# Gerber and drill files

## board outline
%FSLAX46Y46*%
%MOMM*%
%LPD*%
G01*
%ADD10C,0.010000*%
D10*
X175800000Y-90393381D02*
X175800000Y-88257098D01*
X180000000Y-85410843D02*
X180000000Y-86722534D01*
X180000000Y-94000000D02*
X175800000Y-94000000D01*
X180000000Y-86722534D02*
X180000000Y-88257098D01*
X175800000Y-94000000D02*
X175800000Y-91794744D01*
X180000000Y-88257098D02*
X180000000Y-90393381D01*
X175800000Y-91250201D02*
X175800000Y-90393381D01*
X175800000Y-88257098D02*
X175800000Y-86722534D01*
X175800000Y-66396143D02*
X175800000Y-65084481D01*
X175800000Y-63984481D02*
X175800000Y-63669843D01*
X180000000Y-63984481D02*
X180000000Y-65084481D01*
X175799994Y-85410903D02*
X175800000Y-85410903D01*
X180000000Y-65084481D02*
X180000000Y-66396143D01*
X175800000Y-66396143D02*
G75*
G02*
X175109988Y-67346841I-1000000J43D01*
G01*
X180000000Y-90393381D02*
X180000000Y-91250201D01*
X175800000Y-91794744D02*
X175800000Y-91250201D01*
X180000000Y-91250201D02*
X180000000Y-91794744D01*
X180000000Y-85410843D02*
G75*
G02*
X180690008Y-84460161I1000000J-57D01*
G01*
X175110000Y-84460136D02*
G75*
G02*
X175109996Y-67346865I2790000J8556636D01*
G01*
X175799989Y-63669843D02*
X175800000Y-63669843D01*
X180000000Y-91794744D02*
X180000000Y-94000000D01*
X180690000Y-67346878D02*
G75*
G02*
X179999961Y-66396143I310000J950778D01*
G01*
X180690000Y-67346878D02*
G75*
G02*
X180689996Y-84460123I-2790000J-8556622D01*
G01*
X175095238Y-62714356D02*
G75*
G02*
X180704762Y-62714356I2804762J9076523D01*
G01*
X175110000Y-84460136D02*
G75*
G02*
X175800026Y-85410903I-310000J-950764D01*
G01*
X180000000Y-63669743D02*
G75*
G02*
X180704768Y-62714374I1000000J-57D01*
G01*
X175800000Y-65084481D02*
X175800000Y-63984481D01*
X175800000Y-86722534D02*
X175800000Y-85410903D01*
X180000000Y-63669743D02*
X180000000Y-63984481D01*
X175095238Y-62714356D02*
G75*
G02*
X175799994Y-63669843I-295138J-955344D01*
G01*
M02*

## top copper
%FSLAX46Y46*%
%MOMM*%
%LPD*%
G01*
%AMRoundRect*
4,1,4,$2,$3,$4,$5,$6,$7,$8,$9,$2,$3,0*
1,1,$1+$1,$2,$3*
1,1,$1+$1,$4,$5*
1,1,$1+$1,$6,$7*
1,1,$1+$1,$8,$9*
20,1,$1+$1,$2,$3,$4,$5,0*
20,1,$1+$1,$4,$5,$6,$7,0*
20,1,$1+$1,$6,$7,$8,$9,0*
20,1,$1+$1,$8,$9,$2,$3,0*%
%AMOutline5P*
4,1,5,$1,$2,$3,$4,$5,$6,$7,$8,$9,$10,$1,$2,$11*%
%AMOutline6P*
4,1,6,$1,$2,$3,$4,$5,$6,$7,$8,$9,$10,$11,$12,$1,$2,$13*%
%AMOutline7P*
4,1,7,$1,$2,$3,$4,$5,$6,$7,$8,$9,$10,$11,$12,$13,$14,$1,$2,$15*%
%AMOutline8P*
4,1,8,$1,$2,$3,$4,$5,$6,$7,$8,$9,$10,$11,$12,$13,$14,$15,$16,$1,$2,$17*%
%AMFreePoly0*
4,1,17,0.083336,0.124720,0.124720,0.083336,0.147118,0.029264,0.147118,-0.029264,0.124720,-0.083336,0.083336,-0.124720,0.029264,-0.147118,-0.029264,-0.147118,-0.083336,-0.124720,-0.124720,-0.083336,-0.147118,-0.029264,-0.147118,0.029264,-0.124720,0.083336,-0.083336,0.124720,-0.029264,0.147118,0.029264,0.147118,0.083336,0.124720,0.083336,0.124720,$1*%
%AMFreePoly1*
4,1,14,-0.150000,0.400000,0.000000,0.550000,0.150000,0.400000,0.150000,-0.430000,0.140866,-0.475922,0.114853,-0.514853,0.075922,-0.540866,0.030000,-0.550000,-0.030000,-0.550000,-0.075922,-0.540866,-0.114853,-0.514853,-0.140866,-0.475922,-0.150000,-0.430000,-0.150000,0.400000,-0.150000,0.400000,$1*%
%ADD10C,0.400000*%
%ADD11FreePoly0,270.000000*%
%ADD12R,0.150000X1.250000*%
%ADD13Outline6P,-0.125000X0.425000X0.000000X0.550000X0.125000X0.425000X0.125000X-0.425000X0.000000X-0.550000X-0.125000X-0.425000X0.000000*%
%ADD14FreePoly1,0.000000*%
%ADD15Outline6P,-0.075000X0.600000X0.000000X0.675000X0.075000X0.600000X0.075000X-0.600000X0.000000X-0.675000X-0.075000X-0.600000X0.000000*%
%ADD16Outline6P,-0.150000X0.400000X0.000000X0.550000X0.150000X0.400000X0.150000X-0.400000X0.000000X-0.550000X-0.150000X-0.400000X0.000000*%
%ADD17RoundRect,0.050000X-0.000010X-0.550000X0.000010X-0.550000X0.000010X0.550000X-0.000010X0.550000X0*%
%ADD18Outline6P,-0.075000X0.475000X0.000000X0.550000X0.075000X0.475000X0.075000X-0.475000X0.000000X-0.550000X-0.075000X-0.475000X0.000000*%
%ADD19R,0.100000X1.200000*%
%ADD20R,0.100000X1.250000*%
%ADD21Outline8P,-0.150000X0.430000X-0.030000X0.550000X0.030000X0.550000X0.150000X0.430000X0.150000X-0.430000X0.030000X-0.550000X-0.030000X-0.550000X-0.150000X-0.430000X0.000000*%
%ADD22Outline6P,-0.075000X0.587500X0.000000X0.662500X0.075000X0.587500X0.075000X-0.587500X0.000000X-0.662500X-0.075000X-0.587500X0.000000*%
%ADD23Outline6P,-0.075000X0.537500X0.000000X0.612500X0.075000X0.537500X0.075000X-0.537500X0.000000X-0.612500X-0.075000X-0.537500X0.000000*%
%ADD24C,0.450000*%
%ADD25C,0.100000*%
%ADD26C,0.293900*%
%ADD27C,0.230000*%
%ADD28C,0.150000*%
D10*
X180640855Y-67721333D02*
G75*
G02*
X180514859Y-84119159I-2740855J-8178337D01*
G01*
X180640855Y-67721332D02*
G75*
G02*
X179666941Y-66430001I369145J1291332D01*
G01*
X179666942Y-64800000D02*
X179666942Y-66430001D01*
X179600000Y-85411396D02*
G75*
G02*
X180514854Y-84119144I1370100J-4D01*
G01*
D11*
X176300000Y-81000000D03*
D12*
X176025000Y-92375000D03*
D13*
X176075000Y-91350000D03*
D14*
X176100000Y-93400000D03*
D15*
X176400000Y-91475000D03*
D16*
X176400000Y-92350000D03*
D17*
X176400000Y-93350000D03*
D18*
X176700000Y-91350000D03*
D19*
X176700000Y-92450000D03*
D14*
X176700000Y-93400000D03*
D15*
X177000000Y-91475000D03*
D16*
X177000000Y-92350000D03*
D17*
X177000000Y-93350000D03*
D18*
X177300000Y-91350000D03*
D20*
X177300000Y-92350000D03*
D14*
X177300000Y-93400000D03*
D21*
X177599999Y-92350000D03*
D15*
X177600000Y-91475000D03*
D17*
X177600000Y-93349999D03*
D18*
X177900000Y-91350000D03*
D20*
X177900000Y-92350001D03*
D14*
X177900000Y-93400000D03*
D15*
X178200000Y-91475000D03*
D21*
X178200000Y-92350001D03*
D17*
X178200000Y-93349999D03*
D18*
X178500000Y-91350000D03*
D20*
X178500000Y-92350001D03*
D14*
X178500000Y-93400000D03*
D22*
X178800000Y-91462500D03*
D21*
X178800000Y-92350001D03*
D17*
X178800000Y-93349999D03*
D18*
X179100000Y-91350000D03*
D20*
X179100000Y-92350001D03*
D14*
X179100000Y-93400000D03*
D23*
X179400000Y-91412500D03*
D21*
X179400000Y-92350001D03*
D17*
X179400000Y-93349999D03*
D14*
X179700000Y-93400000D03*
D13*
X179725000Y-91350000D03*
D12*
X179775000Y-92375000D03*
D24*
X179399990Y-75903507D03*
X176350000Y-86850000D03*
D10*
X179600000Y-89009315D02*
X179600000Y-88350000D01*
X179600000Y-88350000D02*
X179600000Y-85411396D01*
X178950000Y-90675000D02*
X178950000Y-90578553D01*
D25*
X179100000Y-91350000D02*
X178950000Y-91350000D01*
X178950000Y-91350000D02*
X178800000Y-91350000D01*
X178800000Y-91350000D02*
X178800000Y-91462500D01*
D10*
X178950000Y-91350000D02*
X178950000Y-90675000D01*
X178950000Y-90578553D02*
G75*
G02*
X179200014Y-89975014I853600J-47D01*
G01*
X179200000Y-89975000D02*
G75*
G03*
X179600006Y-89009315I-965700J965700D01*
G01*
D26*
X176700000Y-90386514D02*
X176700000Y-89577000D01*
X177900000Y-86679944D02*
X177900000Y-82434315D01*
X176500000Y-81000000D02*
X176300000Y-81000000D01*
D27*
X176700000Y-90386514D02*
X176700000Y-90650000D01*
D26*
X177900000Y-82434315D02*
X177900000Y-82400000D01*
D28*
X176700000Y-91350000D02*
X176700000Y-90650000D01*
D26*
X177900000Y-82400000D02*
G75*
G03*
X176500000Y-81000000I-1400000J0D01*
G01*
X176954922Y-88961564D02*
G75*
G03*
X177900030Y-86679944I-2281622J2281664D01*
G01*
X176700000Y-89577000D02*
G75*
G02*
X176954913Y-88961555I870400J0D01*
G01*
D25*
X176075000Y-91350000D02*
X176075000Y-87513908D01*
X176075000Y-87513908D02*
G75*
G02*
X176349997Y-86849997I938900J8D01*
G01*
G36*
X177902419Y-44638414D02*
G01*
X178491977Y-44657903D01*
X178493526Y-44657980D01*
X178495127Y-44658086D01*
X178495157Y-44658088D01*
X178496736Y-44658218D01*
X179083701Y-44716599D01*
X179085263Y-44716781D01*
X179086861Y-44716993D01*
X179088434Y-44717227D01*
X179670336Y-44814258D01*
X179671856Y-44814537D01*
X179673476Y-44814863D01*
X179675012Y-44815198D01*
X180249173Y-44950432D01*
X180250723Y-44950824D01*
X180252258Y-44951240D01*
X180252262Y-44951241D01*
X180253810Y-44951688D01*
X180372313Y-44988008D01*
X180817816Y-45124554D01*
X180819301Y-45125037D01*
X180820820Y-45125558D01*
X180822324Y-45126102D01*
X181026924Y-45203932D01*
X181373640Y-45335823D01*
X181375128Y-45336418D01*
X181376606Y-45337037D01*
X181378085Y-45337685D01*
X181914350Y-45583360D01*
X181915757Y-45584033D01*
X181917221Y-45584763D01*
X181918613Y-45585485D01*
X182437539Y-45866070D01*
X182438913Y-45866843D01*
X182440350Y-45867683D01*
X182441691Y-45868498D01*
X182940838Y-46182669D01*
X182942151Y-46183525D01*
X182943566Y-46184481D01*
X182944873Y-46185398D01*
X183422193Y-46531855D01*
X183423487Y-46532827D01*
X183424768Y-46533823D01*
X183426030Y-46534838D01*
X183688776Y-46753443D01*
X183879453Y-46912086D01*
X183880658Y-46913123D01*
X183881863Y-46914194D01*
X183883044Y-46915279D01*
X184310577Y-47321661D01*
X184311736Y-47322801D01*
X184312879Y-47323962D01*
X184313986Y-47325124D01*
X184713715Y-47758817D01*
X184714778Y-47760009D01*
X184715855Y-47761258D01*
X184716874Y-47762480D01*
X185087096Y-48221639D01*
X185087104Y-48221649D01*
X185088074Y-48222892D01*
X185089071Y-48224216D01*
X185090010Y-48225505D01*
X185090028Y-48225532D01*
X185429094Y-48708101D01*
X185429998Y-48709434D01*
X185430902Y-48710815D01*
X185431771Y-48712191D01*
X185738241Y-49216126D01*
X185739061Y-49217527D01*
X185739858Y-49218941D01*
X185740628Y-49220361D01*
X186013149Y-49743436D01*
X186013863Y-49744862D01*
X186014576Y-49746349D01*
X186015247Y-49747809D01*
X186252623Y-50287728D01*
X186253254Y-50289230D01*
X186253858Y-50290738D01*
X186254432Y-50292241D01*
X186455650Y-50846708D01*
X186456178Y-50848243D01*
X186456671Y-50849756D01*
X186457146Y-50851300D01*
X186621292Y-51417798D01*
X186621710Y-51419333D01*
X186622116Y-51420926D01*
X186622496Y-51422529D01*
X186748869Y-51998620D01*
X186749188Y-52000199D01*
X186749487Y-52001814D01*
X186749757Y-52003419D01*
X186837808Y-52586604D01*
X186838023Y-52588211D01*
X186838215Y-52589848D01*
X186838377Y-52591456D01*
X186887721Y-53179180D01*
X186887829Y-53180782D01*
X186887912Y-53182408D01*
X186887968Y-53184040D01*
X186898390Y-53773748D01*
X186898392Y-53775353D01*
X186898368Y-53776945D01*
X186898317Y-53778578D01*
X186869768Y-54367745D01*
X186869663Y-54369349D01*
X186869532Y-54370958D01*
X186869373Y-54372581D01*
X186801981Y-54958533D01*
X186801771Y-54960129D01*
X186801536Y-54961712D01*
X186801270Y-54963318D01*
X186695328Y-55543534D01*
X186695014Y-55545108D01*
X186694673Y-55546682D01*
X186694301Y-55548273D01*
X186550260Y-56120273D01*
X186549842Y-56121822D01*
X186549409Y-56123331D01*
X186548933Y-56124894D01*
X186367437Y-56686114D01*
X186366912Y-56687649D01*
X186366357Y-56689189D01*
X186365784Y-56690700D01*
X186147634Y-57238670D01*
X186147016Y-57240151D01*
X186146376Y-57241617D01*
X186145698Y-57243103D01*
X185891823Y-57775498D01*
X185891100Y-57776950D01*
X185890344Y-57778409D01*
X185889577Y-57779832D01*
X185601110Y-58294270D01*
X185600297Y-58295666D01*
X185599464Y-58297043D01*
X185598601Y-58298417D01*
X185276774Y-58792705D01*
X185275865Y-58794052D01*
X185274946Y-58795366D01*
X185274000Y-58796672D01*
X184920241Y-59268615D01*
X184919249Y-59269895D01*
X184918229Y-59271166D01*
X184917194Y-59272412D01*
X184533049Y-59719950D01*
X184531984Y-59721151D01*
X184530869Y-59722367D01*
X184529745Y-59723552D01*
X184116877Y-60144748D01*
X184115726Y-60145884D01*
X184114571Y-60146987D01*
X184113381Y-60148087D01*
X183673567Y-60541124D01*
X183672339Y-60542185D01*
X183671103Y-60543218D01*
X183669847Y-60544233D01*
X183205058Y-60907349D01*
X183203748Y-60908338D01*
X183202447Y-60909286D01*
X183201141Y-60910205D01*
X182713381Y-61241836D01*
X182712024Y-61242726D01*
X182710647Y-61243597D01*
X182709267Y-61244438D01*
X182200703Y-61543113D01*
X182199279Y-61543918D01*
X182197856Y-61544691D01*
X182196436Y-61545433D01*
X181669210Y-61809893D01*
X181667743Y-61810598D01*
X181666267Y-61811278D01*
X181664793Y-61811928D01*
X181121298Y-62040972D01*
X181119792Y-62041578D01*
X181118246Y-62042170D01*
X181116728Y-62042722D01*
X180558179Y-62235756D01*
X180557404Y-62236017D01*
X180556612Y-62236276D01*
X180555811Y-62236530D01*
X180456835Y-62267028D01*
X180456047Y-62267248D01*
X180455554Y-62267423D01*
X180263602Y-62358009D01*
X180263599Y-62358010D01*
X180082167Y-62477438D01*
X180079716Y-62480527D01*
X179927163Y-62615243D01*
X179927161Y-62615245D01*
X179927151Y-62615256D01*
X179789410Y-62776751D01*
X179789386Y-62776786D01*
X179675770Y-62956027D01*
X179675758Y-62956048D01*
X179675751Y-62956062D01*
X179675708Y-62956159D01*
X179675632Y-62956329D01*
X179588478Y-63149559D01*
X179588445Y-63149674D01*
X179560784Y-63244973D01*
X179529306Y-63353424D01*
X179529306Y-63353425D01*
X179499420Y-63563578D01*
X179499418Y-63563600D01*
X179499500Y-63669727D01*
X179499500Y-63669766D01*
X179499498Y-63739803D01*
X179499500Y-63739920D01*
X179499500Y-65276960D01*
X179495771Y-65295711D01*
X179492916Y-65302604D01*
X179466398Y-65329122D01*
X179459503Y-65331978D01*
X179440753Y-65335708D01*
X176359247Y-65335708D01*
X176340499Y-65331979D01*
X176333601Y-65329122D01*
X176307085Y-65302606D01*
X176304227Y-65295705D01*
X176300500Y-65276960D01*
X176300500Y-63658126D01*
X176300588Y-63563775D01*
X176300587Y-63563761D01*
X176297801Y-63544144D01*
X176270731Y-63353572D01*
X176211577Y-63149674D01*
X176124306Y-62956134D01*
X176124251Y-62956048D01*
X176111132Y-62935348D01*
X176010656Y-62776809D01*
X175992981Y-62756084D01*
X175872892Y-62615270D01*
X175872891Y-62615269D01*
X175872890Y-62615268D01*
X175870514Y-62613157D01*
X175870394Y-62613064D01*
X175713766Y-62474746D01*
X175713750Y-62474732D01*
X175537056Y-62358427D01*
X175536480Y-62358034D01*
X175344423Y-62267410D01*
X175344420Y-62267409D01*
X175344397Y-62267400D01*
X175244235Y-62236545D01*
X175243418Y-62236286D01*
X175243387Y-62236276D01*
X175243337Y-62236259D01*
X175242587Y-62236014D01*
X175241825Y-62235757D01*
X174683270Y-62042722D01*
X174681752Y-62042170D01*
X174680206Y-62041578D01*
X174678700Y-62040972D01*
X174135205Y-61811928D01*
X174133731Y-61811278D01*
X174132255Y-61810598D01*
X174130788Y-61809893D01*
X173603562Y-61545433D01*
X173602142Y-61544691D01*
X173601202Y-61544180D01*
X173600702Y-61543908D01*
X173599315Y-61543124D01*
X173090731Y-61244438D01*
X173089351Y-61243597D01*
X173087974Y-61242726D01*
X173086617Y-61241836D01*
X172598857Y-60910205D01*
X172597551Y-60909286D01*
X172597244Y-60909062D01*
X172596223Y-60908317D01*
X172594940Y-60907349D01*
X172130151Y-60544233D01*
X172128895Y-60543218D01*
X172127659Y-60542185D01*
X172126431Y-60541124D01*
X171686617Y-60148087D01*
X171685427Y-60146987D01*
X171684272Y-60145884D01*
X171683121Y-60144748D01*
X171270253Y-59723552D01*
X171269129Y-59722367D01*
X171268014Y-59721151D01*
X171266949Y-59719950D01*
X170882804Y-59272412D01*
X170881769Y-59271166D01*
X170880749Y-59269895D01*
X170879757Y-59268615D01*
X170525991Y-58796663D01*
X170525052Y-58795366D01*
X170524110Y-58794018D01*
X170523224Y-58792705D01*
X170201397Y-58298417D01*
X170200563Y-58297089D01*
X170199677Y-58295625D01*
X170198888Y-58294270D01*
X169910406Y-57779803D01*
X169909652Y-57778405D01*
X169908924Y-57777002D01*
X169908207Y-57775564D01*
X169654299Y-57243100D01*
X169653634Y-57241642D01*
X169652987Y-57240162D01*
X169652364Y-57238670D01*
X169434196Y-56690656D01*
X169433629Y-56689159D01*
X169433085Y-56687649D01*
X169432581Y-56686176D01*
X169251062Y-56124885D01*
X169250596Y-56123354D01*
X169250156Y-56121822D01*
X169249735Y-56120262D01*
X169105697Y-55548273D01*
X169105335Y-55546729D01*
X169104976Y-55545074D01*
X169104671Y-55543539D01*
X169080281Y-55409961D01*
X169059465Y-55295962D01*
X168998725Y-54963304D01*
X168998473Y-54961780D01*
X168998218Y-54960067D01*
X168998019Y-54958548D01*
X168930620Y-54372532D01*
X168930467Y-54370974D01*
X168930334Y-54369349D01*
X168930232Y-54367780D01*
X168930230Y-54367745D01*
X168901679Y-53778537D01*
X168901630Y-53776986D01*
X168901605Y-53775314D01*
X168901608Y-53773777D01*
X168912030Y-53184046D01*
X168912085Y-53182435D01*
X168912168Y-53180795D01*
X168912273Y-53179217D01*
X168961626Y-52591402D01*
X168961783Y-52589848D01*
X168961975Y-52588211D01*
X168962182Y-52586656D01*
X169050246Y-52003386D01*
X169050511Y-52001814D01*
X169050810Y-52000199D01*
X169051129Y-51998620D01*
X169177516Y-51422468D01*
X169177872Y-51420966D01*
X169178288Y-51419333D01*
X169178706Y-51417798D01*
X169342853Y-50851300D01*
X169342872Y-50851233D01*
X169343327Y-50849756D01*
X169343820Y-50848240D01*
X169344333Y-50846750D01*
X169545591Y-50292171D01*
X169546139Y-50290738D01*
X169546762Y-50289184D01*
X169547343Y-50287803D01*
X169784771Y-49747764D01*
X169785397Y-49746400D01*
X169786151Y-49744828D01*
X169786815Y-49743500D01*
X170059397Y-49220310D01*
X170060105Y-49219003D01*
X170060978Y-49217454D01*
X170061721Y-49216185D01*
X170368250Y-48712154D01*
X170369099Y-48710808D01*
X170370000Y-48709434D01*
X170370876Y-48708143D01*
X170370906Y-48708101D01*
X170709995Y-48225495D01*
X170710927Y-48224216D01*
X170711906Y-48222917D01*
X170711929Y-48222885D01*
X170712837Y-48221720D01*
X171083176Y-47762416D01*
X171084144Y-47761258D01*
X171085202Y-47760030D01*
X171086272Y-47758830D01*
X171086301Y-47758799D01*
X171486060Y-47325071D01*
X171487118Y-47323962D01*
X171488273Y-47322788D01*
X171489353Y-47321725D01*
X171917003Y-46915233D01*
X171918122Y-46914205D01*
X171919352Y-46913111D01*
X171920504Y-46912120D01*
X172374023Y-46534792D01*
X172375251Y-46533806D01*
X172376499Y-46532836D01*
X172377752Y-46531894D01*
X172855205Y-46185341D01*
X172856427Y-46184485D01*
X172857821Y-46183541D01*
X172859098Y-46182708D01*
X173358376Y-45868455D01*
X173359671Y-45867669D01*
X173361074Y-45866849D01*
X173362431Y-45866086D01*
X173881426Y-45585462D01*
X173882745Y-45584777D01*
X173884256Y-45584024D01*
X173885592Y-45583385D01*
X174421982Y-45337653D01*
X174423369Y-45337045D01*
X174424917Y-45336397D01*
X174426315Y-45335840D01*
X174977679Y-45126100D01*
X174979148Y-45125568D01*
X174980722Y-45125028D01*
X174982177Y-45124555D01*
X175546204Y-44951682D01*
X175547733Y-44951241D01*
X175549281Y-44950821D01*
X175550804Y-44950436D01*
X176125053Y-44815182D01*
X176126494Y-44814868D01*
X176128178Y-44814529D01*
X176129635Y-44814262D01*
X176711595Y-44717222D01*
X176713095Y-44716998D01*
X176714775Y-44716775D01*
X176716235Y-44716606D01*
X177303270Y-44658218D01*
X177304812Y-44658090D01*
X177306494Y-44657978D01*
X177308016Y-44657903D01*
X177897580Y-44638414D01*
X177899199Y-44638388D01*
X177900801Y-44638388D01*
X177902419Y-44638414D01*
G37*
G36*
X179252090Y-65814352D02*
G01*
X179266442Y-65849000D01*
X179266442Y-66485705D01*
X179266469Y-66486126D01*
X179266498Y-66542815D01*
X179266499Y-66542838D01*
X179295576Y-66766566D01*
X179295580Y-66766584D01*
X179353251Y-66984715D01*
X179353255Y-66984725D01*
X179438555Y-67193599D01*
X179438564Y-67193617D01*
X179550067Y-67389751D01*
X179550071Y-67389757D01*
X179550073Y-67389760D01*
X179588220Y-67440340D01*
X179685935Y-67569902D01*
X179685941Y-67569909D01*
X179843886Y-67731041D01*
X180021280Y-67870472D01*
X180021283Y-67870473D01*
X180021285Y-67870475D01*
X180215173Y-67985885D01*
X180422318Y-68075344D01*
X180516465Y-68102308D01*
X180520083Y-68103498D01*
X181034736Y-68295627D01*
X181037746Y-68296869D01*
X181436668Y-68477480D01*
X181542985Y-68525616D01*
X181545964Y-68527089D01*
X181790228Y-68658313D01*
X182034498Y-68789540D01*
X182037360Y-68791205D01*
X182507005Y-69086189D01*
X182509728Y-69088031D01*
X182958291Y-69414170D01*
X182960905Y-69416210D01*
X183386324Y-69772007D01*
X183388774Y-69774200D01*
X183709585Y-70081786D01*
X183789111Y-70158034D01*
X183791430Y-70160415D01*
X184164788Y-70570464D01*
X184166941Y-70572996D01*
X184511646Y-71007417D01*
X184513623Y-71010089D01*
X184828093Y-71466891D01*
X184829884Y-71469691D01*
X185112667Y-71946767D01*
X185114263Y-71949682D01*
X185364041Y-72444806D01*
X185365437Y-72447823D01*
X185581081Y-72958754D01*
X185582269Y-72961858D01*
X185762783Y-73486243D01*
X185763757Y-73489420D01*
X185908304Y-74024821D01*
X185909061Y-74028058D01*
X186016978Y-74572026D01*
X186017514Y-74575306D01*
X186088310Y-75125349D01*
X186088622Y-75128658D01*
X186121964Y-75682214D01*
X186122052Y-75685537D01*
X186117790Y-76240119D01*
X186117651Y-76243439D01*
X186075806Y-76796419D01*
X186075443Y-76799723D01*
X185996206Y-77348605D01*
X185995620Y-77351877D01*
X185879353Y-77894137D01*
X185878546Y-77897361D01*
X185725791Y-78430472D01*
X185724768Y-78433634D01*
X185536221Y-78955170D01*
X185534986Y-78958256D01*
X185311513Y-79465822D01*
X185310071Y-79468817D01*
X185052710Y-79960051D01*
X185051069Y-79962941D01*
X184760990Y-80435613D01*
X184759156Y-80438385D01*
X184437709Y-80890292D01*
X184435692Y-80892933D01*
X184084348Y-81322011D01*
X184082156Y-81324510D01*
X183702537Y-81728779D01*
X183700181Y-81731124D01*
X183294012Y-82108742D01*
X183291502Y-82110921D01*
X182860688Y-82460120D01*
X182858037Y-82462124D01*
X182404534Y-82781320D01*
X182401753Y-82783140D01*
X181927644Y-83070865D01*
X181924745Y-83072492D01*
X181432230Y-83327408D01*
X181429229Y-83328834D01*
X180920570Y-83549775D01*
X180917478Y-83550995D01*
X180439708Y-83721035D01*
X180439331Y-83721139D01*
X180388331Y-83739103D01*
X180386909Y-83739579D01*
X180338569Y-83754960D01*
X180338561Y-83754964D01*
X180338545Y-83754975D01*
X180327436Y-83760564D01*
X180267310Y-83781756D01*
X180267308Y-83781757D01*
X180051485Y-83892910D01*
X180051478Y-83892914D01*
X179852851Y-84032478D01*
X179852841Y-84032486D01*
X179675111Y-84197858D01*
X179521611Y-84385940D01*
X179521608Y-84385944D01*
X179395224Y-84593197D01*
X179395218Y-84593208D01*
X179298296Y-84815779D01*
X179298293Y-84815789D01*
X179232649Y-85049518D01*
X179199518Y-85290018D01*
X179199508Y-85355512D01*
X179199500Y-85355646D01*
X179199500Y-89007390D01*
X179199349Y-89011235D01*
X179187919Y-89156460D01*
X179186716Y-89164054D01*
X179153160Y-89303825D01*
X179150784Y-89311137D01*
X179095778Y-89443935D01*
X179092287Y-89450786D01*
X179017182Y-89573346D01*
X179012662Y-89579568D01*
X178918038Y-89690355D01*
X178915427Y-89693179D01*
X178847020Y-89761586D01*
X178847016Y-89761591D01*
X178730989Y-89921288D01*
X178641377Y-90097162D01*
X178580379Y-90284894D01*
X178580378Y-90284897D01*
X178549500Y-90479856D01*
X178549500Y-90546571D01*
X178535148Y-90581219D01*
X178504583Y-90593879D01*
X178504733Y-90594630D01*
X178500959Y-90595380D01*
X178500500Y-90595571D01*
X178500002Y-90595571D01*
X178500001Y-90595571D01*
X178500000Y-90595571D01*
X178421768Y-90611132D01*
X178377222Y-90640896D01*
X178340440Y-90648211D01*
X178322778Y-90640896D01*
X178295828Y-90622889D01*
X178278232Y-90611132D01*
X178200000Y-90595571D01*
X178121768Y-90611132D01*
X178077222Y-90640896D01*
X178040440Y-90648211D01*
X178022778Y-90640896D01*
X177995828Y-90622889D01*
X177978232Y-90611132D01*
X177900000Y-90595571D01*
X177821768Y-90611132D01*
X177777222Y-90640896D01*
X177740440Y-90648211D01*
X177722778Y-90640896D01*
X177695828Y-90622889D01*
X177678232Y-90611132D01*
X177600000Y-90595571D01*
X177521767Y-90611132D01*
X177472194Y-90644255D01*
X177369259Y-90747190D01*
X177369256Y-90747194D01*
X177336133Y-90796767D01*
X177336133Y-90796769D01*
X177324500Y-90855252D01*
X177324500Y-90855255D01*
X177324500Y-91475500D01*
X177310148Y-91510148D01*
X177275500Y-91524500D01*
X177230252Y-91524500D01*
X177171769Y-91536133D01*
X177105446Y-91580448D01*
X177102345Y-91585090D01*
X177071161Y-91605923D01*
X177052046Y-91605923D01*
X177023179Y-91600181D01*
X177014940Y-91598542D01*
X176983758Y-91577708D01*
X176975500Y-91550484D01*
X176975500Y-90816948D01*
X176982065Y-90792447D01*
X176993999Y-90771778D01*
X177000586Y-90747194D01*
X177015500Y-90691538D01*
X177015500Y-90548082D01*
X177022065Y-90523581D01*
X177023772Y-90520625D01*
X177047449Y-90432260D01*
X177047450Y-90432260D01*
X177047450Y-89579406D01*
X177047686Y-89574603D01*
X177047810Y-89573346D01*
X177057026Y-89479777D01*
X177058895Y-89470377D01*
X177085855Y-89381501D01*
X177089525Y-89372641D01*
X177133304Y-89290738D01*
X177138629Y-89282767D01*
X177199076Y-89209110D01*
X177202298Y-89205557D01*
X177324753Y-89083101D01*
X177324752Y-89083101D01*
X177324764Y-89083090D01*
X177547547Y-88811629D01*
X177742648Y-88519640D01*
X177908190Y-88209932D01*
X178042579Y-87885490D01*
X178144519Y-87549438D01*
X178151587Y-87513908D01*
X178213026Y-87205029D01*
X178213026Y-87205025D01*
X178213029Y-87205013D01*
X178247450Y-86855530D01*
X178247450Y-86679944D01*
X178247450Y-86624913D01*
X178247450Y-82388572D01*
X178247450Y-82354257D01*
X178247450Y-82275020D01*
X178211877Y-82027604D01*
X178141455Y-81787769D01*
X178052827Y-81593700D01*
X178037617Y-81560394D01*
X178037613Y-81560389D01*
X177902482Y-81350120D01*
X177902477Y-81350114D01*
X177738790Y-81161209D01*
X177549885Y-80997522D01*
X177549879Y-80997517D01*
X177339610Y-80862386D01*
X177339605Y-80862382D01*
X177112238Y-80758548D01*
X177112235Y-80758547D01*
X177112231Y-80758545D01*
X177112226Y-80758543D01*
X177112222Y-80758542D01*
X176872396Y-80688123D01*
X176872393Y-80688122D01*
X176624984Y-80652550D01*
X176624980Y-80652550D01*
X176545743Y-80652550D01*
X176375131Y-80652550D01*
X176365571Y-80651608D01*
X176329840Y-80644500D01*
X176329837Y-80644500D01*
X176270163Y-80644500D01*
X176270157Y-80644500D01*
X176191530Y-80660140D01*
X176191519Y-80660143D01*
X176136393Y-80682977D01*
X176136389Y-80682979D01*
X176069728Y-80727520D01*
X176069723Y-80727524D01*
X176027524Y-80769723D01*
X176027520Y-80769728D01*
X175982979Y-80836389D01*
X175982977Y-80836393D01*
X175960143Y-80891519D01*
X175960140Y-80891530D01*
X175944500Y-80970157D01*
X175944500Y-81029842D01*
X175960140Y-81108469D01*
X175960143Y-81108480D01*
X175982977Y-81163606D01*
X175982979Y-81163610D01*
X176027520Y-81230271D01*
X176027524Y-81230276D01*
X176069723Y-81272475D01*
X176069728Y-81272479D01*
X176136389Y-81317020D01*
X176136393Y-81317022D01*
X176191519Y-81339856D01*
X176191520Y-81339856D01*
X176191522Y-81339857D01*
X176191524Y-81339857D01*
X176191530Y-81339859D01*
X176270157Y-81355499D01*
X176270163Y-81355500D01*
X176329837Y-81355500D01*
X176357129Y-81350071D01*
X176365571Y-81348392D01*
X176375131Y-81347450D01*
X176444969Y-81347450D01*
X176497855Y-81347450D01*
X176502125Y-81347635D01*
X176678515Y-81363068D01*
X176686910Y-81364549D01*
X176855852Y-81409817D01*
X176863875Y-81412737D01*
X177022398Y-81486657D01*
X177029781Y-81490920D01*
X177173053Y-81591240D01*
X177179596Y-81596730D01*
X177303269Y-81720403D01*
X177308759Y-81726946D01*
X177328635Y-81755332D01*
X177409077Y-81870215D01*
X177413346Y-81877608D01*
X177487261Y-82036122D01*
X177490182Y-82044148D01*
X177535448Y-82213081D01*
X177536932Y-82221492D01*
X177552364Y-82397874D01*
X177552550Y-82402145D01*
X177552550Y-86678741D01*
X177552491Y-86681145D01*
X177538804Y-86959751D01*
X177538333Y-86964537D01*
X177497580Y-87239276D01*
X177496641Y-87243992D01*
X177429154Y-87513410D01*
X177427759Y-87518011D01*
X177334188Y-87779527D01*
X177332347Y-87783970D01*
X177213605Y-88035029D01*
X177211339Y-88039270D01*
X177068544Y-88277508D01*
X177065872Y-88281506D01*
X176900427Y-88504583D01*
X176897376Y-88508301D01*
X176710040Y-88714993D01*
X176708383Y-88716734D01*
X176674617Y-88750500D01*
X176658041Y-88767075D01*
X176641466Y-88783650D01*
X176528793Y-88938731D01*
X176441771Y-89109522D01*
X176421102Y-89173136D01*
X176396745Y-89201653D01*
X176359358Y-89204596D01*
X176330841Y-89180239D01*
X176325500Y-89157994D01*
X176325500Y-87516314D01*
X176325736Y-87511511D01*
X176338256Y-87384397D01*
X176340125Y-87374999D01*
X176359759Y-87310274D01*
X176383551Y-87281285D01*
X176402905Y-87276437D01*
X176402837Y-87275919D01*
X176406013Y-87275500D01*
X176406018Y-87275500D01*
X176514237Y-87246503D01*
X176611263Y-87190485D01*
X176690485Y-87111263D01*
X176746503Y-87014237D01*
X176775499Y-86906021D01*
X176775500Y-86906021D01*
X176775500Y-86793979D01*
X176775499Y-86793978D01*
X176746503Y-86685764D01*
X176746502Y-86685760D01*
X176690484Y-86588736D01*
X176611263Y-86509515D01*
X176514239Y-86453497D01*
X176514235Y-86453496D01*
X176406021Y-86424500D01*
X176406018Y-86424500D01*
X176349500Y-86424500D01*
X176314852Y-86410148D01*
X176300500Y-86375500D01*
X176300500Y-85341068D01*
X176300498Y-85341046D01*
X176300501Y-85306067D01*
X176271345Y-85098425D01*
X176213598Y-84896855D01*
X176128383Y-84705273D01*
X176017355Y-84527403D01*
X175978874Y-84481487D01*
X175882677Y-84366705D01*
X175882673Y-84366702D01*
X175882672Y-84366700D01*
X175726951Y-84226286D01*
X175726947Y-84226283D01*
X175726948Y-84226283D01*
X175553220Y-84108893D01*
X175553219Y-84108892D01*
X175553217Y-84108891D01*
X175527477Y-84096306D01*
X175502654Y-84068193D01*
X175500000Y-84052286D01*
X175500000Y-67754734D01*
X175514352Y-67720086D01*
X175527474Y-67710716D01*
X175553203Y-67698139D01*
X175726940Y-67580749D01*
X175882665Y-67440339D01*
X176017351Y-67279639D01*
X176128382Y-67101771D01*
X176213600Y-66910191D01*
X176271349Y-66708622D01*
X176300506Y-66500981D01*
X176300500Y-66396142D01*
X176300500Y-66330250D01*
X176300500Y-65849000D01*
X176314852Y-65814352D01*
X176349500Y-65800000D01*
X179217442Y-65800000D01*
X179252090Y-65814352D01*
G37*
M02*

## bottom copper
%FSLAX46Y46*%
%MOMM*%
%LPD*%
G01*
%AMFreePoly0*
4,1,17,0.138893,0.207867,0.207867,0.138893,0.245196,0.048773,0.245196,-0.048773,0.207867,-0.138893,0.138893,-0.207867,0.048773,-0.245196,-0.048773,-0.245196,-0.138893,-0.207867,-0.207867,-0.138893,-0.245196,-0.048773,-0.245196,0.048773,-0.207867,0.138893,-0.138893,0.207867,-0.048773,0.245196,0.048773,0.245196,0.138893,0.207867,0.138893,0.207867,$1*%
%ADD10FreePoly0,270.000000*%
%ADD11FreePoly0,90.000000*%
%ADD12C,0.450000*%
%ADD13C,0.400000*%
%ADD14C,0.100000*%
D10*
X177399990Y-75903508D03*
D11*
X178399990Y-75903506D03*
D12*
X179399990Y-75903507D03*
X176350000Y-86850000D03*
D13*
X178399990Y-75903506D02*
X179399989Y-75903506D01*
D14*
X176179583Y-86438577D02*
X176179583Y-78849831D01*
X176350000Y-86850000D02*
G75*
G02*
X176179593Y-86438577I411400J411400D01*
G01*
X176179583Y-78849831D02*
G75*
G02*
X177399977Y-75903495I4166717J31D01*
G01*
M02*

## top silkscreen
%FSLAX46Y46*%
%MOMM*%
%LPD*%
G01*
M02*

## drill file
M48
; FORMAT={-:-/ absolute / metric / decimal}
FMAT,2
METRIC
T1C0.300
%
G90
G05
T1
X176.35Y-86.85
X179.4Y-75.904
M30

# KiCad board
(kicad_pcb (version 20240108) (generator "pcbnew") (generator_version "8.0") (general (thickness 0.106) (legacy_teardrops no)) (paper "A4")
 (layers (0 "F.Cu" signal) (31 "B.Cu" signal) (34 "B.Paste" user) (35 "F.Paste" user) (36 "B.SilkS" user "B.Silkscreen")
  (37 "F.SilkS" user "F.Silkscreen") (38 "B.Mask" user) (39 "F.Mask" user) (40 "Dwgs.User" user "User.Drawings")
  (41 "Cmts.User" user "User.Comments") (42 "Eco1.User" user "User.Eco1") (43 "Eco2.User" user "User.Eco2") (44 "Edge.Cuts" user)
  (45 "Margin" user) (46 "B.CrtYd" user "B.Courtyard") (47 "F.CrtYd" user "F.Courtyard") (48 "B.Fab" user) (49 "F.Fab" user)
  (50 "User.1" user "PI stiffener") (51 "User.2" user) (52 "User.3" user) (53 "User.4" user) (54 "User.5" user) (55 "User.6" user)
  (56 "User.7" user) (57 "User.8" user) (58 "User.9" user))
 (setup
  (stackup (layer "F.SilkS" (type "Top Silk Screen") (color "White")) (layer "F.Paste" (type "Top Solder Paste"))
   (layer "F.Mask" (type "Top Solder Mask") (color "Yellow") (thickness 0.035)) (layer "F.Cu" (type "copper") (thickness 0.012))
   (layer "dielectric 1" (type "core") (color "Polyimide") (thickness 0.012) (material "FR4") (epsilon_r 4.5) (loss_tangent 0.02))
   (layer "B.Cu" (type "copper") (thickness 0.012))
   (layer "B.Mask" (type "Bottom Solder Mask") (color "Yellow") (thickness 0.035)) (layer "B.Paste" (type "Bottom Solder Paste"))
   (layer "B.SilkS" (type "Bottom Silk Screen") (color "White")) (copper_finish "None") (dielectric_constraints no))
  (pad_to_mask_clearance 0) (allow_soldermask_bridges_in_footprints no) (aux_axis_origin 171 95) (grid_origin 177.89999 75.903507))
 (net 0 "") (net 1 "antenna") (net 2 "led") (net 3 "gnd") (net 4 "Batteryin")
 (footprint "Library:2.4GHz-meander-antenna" (layer "F.Cu") (at 176.3 81 -90)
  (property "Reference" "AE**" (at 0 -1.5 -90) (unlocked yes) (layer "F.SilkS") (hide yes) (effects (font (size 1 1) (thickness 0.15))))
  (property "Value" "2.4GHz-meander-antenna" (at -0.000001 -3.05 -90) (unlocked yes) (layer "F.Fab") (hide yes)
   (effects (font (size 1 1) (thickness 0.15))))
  (pad "1" smd custom (at 0 0 270) (size 0.3 0.3) (layers "F.Cu") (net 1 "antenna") (thermal_bridge_angle 90)
   (options (clearance outline) (anchor circle)) (primitives)))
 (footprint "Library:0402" (layer "B.Cu") (at 177.89999 75.903507)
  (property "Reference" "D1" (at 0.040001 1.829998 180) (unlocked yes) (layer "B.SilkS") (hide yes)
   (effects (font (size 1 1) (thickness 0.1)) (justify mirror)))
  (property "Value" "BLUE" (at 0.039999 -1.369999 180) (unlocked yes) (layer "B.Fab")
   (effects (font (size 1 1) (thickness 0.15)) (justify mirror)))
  (pad "1" smd custom (at -0.5 0.000001 270) (size 0.5 0.5) (layers "B.Cu" "B.Paste" "B.Mask") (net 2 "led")
   (options (clearance outline) (anchor circle)) (primitives))
  (pad "2" smd custom (at 0.5 -0.000001 90) (size 0.5 0.5) (layers "B.Cu" "B.Paste" "B.Mask") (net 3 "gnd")
   (options (clearance outline) (anchor circle)) (primitives)))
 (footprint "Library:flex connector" (layer "B.Cu") (at 175.7 90.05)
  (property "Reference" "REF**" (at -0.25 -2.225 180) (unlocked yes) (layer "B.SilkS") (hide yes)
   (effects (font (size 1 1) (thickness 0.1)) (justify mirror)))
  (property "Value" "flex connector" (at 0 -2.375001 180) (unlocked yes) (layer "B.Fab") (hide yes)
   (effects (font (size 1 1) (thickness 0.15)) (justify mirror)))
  (pad "1" smd rect (at 0.325 2.325) (size 0.15 1.25) (layers "F.Cu" "F.Paste" "F.Mask") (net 2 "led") (thermal_bridge_angle 45))
  (pad "1" smd roundrect (at 0.375 1.3) (size 0.25 1.1) (layers "F.Cu" "F.Paste" "F.Mask") (roundrect_rratio 0) (chamfer_ratio 0.5)
   (chamfer top_left top_right bottom_left bottom_right) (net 2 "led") (thermal_bridge_angle 45))
  (pad "1" smd roundrect (at 0.4 3.35) (size 0.3 1.1) (layers "F.Cu" "F.Paste" "F.Mask") (roundrect_rratio 0.4) (chamfer_ratio 0.5)
   (chamfer top_left top_right) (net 2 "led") (thermal_bridge_angle 45))
  (pad "2" smd roundrect (at 0.7 1.425) (size 0.15 1.35) (layers "F.Cu" "F.Paste" "F.Mask") (roundrect_rratio 0) (chamfer_ratio 0.5)
   (chamfer top_left top_right bottom_left bottom_right) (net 3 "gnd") (thermal_bridge_angle 45))
  (pad "2" smd roundrect (at 0.7 2.3) (size 0.3 1.1) (layers "F.Cu" "F.Paste" "F.Mask") (roundrect_rratio 0) (chamfer_ratio 0.5)
   (chamfer top_left top_right bottom_left bottom_right) (thermal_bridge_angle 45))
  (pad "2" smd roundrect (at 0.7 3.3) (size 0.1 1.2) (layers "F.Cu" "F.Paste" "F.Mask") (roundrect_rratio 0.5) (thermal_bridge_angle 45))
  (pad "3" smd roundrect (at 1 1.3) (size 0.15 1.1) (layers "F.Cu" "F.Paste" "F.Mask") (roundrect_rratio 0) (chamfer_ratio 0.5)
   (chamfer top_left top_right bottom_left bottom_right) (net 1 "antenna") (thermal_bridge_angle 45))
  (pad "3" smd rect (at 1 2.4) (size 0.1 1.2) (layers "F.Cu" "F.Paste" "F.Mask") (thermal_bridge_angle 45))
  (pad "3" smd roundrect (at 1 3.35) (size 0.3 1.1) (layers "F.Cu" "F.Paste" "F.Mask") (roundrect_rratio 0.4) (chamfer_ratio 0.5)
   (chamfer top_left top_right) (thermal_bridge_angle 45))
  (pad "4" smd roundrect (at 1.3 1.425) (size 0.15 1.35) (layers "F.Cu" "F.Paste" "F.Mask") (roundrect_rratio 0) (chamfer_ratio 0.5)
   (chamfer top_left top_right bottom_left bottom_right) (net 3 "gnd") (thermal_bridge_angle 45))
  (pad "4" smd roundrect (at 1.3 2.3) (size 0.3 1.1) (layers "F.Cu" "F.Paste" "F.Mask") (roundrect_rratio 0) (chamfer_ratio 0.5)
   (chamfer top_left top_right bottom_left bottom_right) (thermal_bridge_angle 45))
  (pad "4" smd roundrect (at 1.3 3.3) (size 0.1 1.2) (layers "F.Cu" "F.Paste" "F.Mask") (roundrect_rratio 0.5) (thermal_bridge_angle 45))
  (pad "5" smd roundrect (at 1.6 1.3) (size 0.15 1.1) (layers "F.Cu" "F.Paste" "F.Mask") (roundrect_rratio 0) (chamfer_ratio 0.5)
   (chamfer top_left top_right bottom_left bottom_right) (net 3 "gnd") (thermal_bridge_angle 45))
  (pad "5" smd rect (at 1.6 2.3) (size 0.1 1.25) (layers "F.Cu" "F.Paste" "F.Mask") (thermal_bridge_angle 45))
  (pad "5" smd roundrect (at 1.6 3.35) (size 0.3 1.1) (layers "F.Cu" "F.Paste" "F.Mask") (roundrect_rratio 0.4) (chamfer_ratio 0.5)
   (chamfer top_left top_right) (thermal_bridge_angle 45))
  (pad "6" smd roundrect (at 1.899999 2.3) (size 0.3 1.1) (layers "F.Cu" "F.Paste" "F.Mask") (roundrect_rratio 0) (chamfer_ratio 0.4)
   (chamfer top_left top_right bottom_left bottom_right) (thermal_bridge_angle 45))
  (pad "6" smd roundrect (at 1.9 1.425) (size 0.15 1.35) (layers "F.Cu" "F.Paste" "F.Mask") (roundrect_rratio 0) (chamfer_ratio 0.5)
   (chamfer top_left top_right bottom_left bottom_right) (thermal_bridge_angle 45))
  (pad "6" smd roundrect (at 1.9 3.299999) (size 0.1 1.2) (layers "F.Cu" "F.Paste" "F.Mask") (roundrect_rratio 0.5)
   (thermal_bridge_angle 45))
  (pad "7" smd roundrect (at 2.2 1.3) (size 0.15 1.1) (layers "F.Cu" "F.Paste" "F.Mask") (roundrect_rratio 0) (chamfer_ratio 0.5)
   (chamfer top_left top_right bottom_left bottom_right) (thermal_bridge_angle 45))
  (pad "7" smd rect (at 2.2 2.300001) (size 0.1 1.25) (layers "F.Cu" "F.Paste" "F.Mask") (thermal_bridge_angle 45))
  (pad "7" smd roundrect (at 2.2 3.35) (size 0.3 1.1) (layers "F.Cu" "F.Paste" "F.Mask") (roundrect_rratio 0.4) (chamfer_ratio 0.5)
   (chamfer top_left top_right) (thermal_bridge_angle 45))
  (pad "8" smd roundrect (at 2.5 1.425) (size 0.15 1.35) (layers "F.Cu" "F.Paste" "F.Mask") (roundrect_rratio 0) (chamfer_ratio 0.5)
   (chamfer top_left top_right bottom_left bottom_right) (thermal_bridge_angle 45))
  (pad "8" smd roundrect (at 2.5 2.300001) (size 0.3 1.1) (layers "F.Cu" "F.Paste" "F.Mask") (roundrect_rratio 0) (chamfer_ratio 0.4)
   (chamfer top_left top_right bottom_left bottom_right) (thermal_bridge_angle 45))
  (pad "8" smd roundrect (at 2.5 3.299999) (size 0.1 1.2) (layers "F.Cu" "F.Paste" "F.Mask") (roundrect_rratio 0.5)
   (thermal_bridge_angle 45))
  (pad "9" smd roundrect (at 2.8 1.3) (size 0.15 1.1) (layers "F.Cu" "F.Paste" "F.Mask") (roundrect_rratio 0) (chamfer_ratio 0.5)
   (chamfer top_left top_right bottom_left bottom_right) (thermal_bridge_angle 45))
  (pad "9" smd rect (at 2.8 2.300001) (size 0.1 1.25) (layers "F.Cu" "F.Paste" "F.Mask") (thermal_bridge_angle 45))
  (pad "9" smd roundrect (at 2.8 3.35) (size 0.3 1.1) (layers "F.Cu" "F.Paste" "F.Mask") (roundrect_rratio 0.4) (chamfer_ratio 0.5)
   (chamfer top_left top_right) (thermal_bridge_angle 45))
  (pad "10" smd roundrect (at 3.1 1.4125) (size 0.15 1.325) (layers "F.Cu" "F.Paste" "F.Mask") (roundrect_rratio 0) (chamfer_ratio 0.5)
   (chamfer top_left top_right bottom_left bottom_right) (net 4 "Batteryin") (thermal_bridge_angle 45))
  (pad "10" smd roundrect (at 3.1 2.300001) (size 0.3 1.1) (layers "F.Cu" "F.Paste" "F.Mask") (roundrect_rratio 0) (chamfer_ratio 0.4)
   (chamfer top_left top_right bottom_left bottom_right) (thermal_bridge_angle 45))
  (pad "10" smd roundrect (at 3.1 3.299999) (size 0.1 1.2) (layers "F.Cu" "F.Paste" "F.Mask") (roundrect_rratio 0.5)
   (thermal_bridge_angle 45))
  (pad "11" smd roundrect (at 3.4 1.3) (size 0.15 1.1) (layers "F.Cu" "F.Paste" "F.Mask") (roundrect_rratio 0) (chamfer_ratio 0.5)
   (chamfer top_left top_right bottom_left bottom_right) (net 4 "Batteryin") (thermal_bridge_angle 45))
  (pad "11" smd rect (at 3.4 2.300001) (size 0.1 1.25) (layers "F.Cu" "F.Paste" "F.Mask") (thermal_bridge_angle 45))
  (pad "11" smd roundrect (at 3.4 3.35) (size 0.3 1.1) (layers "F.Cu" "F.Paste" "F.Mask") (roundrect_rratio 0.4) (chamfer_ratio 0.5)
   (chamfer top_left top_right) (thermal_bridge_angle 45))
  (pad "12" smd roundrect (at 3.7 1.3625) (size 0.15 1.225) (layers "F.Cu" "F.Paste" "F.Mask") (roundrect_rratio 0) (chamfer_ratio 0.5)
   (chamfer top_left top_right bottom_left bottom_right) (thermal_bridge_angle 45))
  (pad "12" smd roundrect (at 3.7 2.300001) (size 0.3 1.1) (layers "F.Cu" "F.Paste" "F.Mask") (roundrect_rratio 0) (chamfer_ratio 0.4)
   (chamfer top_left top_right bottom_left bottom_right) (thermal_bridge_angle 45))
  (pad "12" smd roundrect (at 3.7 3.299999) (size 0.1 1.2) (layers "F.Cu" "F.Paste" "F.Mask") (roundrect_rratio 0.5)
   (thermal_bridge_angle 45))
  (pad "13" smd roundrect (at 4 3.35) (size 0.3 1.1) (layers "F.Cu" "F.Paste" "F.Mask") (roundrect_rratio 0.4) (chamfer_ratio 0.5)
   (chamfer top_left top_right) (thermal_bridge_angle 45))
  (pad "13" smd roundrect (at 4.025 1.3) (size 0.25 1.1) (layers "F.Cu" "F.Paste" "F.Mask") (roundrect_rratio 0) (chamfer_ratio 0.5)
   (chamfer top_left top_right bottom_left bottom_right) (thermal_bridge_angle 45))
  (pad "13" smd rect (at 4.075 2.325) (size 0.15 1.25) (layers "F.Cu" "F.Paste" "F.Mask") (thermal_bridge_angle 45)))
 (gr_arc (start 180.640855 67.721333) (mid 186.525141 75.965942) (end 180.514858 84.119155) (stroke (width 0.4) (type default))
  (layer "F.Cu") (net 4))
 (gr_arc (start 180.640855 67.721332) (mid 179.937716 67.23871) (end 179.666942 66.430001) (stroke (width 0.4) (type default))
  (layer "F.Cu") (net 4))
 (gr_line (start 179.666942 64.8) (end 179.666942 66.430001) (stroke (width 0.4) (type default)) (layer "F.Cu") (net 4))
 (gr_arc (start 179.6 85.411396) (mid 179.851865 84.619744) (end 180.514858 84.119156) (stroke (width 0.4) (type default)) (layer "F.Cu")
  (net 4))
 (gr_line (start 175.8 90.393381) (end 175.8 88.257098) (stroke (width 0.01) (type default)) (layer "Edge.Cuts"))
 (gr_line (start 180 85.410843) (end 180 86.722534) (stroke (width 0.01) (type default)) (layer "Edge.Cuts"))
 (gr_line (start 180 94) (end 175.8 94) (stroke (width 0.01) (type default)) (layer "Edge.Cuts"))
 (gr_line (start 180 86.722534) (end 180 88.257098) (stroke (width 0.01) (type default)) (layer "Edge.Cuts"))
 (gr_line (start 175.8 94) (end 175.8 91.794744) (stroke (width 0.01) (type default)) (layer "Edge.Cuts"))
 (gr_line (start 180 88.257098) (end 180 90.393381) (stroke (width 0.01) (type default)) (layer "Edge.Cuts"))
 (gr_line (start 175.8 91.250201) (end 175.8 90.393381) (stroke (width 0.01) (type default)) (layer "Edge.Cuts"))
 (gr_line (start 175.8 88.257098) (end 175.8 86.722534) (stroke (width 0.01) (type default)) (layer "Edge.Cuts"))
 (gr_line (start 175.8 66.396143) (end 175.8 65.084481) (stroke (width 0.01) (type default)) (layer "Edge.Cuts"))
 (gr_line (start 175.8 63.984481) (end 175.8 63.669843) (stroke (width 0.01) (type default)) (layer "Edge.Cuts"))
 (gr_line (start 180 63.984481) (end 180 65.084481) (stroke (width 0.01) (type default)) (layer "Edge.Cuts"))
 (gr_line (start 175.799994 85.410903) (end 175.8 85.410903) (stroke (width 0.01) (type default)) (layer "Edge.Cuts"))
 (gr_line (start 180 65.084481) (end 180 66.396143) (stroke (width 0.01) (type default)) (layer "Edge.Cuts"))
 (gr_arc (start 175.8 66.396143) (mid 175.609321 66.98351) (end 175.11 67.346878) (stroke (width 0.01) (type default)) (layer "Edge.Cuts"))
 (gr_line (start 180 90.393381) (end 180 91.250201) (stroke (width 0.01) (type default)) (layer "Edge.Cuts"))
 (gr_line (start 175.8 91.794744) (end 175.8 91.250201) (stroke (width 0.01) (type default)) (layer "Edge.Cuts"))
 (gr_line (start 180 91.250201) (end 180 91.794744) (stroke (width 0.01) (type default)) (layer "Edge.Cuts"))
 (gr_arc (start 180 85.410843) (mid 180.190685 84.8235) (end 180.69 84.460136) (stroke (width 0.01) (type default)) (layer "Edge.Cuts"))
 (gr_arc (start 175.11 84.460136) (mid 168.9 75.903507) (end 175.11 67.346878) (stroke (width 0.01) (type default)) (layer "Edge.Cuts"))
 (gr_line (start 175.799989 63.669843) (end 175.8 63.669843) (stroke (width 0.01) (type default)) (layer "Edge.Cuts"))
 (gr_line (start 180 91.794744) (end 180 94) (stroke (width 0.01) (type default)) (layer "Edge.Cuts"))
 (gr_arc (start 180.69 67.346878) (mid 180.19068 66.983509) (end 180 66.396143) (stroke (width 0.01) (type default)) (layer "Edge.Cuts"))
 (gr_arc (start 180.69 67.346878) (mid 186.9 75.903507) (end 180.69 84.460136) (stroke (width 0.01) (type default)) (layer "Edge.Cuts"))
 (gr_arc (start 175.095238 62.714356) (mid 177.9 44.137835) (end 180.704762 62.714356) (stroke (width 0.01) (type default))
  (layer "Edge.Cuts"))
 (gr_arc (start 175.11 84.460136) (mid 175.609319 84.823524) (end 175.799994 85.410903) (stroke (width 0.01) (type default))
  (layer "Edge.Cuts"))
 (gr_arc (start 180 63.669743) (mid 180.195258 63.076151) (end 180.704762 62.714356) (stroke (width 0.01) (type default))
  (layer "Edge.Cuts"))
 (gr_line (start 175.8 65.084481) (end 175.8 63.984481) (stroke (width 0.01) (type default)) (layer "Edge.Cuts"))
 (gr_line (start 175.8 86.722534) (end 175.8 85.410903) (stroke (width 0.01) (type default)) (layer "Edge.Cuts"))
 (gr_line (start 180 63.669743) (end 180 63.984481) (stroke (width 0.01) (type default)) (layer "Edge.Cuts"))
 (gr_arc (start 175.095238 62.714356) (mid 175.604791 63.076183) (end 175.799989 63.669843) (stroke (width 0.01) (type default))
  (layer "Edge.Cuts"))
 (segment (start 179.6 89.009315) (end 179.6 88.35) (width 0.4) (layer "F.Cu") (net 4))
 (segment (start 179.6 88.35) (end 179.6 85.411396) (width 0.4) (layer "F.Cu") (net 4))
 (segment (start 178.95 90.675) (end 178.95 90.578553) (width 0.4) (layer "F.Cu") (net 4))
 (segment (start 179.1 91.35) (end 178.95 91.35) (width 0.1) (layer "F.Cu") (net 4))
 (segment (start 178.95 91.35) (end 178.8 91.35) (width 0.1) (layer "F.Cu") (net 4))
 (segment (start 178.8 91.35) (end 178.8 91.4625) (width 0.1) (layer "F.Cu") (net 4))
 (segment (start 178.95 91.35) (end 178.95 90.675) (width 0.4) (layer "F.Cu") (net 4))
 (arc (start 178.95 90.578553) (mid 179.014973 90.251913) (end 179.2 89.975) (width 0.4) (layer "F.Cu") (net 4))
 (arc (start 179.2 89.975) (mid 179.496044 89.53194) (end 179.6 89.009315) (width 0.4) (layer "F.Cu") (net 4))
 (via (at 179.39999 75.903507) (size 0.45) (drill 0.3) (layers "F.Cu" "B.Cu") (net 3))
 (segment (start 178.39999 75.903506) (end 179.399989 75.903506) (width 0.4) (layer "B.Cu") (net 3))
 (segment (start 176.7 90.386514) (end 176.7 89.577) (width 0.2939) (layer "F.Cu") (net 1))
 (segment (start 177.9 86.679944) (end 177.9 82.434315) (width 0.2939) (layer "F.Cu") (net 1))
 (segment (start 176.5 81) (end 176.3 81) (width 0.2939) (layer "F.Cu") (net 1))
 (segment (start 176.7 90.386514) (end 176.7 90.65) (width 0.23) (layer "F.Cu") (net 1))
 (segment (start 177.9 82.434315) (end 177.9 82.4) (width 0.2939) (layer "F.Cu") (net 1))
 (segment (start 176.7 91.35) (end 176.7 90.65) (width 0.15) (layer "F.Cu") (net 1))
 (arc (start 177.9 82.4) (mid 177.489949 81.410051) (end 176.5 81) (width 0.2939) (layer "F.Cu") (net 1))
 (arc (start 176.954922 88.961564) (mid 177.654383 87.914748) (end 177.9 86.679944) (width 0.2939) (layer "F.Cu") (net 1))
 (arc (start 176.7 89.577) (mid 176.766252 89.243929) (end 176.954922 88.961564) (width 0.2939) (layer "F.Cu") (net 1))
 (segment (start 176.075 91.35) (end 176.075 87.513908) (width 0.1) (layer "F.Cu") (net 2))
 (via (at 176.35 86.85) (size 0.45) (drill 0.3) (layers "F.Cu" "B.Cu") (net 2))
 (arc (start 176.075 87.513908) (mid 176.14647 87.154604) (end 176.35 86.85) (width 0.1) (layer "F.Cu") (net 2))
 (segment (start 176.179583 86.438577) (end 176.179583 78.849831) (width 0.1) (layer "B.Cu") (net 2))
 (arc (start 176.35 86.85) (mid 176.223873 86.661237) (end 176.179583 86.438577) (width 0.1) (layer "B.Cu") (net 2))
 (arc (start 176.179583 78.849831) (mid 176.496756 77.255293) (end 177.39999 75.903508) (width 0.1) (layer "B.Cu") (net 2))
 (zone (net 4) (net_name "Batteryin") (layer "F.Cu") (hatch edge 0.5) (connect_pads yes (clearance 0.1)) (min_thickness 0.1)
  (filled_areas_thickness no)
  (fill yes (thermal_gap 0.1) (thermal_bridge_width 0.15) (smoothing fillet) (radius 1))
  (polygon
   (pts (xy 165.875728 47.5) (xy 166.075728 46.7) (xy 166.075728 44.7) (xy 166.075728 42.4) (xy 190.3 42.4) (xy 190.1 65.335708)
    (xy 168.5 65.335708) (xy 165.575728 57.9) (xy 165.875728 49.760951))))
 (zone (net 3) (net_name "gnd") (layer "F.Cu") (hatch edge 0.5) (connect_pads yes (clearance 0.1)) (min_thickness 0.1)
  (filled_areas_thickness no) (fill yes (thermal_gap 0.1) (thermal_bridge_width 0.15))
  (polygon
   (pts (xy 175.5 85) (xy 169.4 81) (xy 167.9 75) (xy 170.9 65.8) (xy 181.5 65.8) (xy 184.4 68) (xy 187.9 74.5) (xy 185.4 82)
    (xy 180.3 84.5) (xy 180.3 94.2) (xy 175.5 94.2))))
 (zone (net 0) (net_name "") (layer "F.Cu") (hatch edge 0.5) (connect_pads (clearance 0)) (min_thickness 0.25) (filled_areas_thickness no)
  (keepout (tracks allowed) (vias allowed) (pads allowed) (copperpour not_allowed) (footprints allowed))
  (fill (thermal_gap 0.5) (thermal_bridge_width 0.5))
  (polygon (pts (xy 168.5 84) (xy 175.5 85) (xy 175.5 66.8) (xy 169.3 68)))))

